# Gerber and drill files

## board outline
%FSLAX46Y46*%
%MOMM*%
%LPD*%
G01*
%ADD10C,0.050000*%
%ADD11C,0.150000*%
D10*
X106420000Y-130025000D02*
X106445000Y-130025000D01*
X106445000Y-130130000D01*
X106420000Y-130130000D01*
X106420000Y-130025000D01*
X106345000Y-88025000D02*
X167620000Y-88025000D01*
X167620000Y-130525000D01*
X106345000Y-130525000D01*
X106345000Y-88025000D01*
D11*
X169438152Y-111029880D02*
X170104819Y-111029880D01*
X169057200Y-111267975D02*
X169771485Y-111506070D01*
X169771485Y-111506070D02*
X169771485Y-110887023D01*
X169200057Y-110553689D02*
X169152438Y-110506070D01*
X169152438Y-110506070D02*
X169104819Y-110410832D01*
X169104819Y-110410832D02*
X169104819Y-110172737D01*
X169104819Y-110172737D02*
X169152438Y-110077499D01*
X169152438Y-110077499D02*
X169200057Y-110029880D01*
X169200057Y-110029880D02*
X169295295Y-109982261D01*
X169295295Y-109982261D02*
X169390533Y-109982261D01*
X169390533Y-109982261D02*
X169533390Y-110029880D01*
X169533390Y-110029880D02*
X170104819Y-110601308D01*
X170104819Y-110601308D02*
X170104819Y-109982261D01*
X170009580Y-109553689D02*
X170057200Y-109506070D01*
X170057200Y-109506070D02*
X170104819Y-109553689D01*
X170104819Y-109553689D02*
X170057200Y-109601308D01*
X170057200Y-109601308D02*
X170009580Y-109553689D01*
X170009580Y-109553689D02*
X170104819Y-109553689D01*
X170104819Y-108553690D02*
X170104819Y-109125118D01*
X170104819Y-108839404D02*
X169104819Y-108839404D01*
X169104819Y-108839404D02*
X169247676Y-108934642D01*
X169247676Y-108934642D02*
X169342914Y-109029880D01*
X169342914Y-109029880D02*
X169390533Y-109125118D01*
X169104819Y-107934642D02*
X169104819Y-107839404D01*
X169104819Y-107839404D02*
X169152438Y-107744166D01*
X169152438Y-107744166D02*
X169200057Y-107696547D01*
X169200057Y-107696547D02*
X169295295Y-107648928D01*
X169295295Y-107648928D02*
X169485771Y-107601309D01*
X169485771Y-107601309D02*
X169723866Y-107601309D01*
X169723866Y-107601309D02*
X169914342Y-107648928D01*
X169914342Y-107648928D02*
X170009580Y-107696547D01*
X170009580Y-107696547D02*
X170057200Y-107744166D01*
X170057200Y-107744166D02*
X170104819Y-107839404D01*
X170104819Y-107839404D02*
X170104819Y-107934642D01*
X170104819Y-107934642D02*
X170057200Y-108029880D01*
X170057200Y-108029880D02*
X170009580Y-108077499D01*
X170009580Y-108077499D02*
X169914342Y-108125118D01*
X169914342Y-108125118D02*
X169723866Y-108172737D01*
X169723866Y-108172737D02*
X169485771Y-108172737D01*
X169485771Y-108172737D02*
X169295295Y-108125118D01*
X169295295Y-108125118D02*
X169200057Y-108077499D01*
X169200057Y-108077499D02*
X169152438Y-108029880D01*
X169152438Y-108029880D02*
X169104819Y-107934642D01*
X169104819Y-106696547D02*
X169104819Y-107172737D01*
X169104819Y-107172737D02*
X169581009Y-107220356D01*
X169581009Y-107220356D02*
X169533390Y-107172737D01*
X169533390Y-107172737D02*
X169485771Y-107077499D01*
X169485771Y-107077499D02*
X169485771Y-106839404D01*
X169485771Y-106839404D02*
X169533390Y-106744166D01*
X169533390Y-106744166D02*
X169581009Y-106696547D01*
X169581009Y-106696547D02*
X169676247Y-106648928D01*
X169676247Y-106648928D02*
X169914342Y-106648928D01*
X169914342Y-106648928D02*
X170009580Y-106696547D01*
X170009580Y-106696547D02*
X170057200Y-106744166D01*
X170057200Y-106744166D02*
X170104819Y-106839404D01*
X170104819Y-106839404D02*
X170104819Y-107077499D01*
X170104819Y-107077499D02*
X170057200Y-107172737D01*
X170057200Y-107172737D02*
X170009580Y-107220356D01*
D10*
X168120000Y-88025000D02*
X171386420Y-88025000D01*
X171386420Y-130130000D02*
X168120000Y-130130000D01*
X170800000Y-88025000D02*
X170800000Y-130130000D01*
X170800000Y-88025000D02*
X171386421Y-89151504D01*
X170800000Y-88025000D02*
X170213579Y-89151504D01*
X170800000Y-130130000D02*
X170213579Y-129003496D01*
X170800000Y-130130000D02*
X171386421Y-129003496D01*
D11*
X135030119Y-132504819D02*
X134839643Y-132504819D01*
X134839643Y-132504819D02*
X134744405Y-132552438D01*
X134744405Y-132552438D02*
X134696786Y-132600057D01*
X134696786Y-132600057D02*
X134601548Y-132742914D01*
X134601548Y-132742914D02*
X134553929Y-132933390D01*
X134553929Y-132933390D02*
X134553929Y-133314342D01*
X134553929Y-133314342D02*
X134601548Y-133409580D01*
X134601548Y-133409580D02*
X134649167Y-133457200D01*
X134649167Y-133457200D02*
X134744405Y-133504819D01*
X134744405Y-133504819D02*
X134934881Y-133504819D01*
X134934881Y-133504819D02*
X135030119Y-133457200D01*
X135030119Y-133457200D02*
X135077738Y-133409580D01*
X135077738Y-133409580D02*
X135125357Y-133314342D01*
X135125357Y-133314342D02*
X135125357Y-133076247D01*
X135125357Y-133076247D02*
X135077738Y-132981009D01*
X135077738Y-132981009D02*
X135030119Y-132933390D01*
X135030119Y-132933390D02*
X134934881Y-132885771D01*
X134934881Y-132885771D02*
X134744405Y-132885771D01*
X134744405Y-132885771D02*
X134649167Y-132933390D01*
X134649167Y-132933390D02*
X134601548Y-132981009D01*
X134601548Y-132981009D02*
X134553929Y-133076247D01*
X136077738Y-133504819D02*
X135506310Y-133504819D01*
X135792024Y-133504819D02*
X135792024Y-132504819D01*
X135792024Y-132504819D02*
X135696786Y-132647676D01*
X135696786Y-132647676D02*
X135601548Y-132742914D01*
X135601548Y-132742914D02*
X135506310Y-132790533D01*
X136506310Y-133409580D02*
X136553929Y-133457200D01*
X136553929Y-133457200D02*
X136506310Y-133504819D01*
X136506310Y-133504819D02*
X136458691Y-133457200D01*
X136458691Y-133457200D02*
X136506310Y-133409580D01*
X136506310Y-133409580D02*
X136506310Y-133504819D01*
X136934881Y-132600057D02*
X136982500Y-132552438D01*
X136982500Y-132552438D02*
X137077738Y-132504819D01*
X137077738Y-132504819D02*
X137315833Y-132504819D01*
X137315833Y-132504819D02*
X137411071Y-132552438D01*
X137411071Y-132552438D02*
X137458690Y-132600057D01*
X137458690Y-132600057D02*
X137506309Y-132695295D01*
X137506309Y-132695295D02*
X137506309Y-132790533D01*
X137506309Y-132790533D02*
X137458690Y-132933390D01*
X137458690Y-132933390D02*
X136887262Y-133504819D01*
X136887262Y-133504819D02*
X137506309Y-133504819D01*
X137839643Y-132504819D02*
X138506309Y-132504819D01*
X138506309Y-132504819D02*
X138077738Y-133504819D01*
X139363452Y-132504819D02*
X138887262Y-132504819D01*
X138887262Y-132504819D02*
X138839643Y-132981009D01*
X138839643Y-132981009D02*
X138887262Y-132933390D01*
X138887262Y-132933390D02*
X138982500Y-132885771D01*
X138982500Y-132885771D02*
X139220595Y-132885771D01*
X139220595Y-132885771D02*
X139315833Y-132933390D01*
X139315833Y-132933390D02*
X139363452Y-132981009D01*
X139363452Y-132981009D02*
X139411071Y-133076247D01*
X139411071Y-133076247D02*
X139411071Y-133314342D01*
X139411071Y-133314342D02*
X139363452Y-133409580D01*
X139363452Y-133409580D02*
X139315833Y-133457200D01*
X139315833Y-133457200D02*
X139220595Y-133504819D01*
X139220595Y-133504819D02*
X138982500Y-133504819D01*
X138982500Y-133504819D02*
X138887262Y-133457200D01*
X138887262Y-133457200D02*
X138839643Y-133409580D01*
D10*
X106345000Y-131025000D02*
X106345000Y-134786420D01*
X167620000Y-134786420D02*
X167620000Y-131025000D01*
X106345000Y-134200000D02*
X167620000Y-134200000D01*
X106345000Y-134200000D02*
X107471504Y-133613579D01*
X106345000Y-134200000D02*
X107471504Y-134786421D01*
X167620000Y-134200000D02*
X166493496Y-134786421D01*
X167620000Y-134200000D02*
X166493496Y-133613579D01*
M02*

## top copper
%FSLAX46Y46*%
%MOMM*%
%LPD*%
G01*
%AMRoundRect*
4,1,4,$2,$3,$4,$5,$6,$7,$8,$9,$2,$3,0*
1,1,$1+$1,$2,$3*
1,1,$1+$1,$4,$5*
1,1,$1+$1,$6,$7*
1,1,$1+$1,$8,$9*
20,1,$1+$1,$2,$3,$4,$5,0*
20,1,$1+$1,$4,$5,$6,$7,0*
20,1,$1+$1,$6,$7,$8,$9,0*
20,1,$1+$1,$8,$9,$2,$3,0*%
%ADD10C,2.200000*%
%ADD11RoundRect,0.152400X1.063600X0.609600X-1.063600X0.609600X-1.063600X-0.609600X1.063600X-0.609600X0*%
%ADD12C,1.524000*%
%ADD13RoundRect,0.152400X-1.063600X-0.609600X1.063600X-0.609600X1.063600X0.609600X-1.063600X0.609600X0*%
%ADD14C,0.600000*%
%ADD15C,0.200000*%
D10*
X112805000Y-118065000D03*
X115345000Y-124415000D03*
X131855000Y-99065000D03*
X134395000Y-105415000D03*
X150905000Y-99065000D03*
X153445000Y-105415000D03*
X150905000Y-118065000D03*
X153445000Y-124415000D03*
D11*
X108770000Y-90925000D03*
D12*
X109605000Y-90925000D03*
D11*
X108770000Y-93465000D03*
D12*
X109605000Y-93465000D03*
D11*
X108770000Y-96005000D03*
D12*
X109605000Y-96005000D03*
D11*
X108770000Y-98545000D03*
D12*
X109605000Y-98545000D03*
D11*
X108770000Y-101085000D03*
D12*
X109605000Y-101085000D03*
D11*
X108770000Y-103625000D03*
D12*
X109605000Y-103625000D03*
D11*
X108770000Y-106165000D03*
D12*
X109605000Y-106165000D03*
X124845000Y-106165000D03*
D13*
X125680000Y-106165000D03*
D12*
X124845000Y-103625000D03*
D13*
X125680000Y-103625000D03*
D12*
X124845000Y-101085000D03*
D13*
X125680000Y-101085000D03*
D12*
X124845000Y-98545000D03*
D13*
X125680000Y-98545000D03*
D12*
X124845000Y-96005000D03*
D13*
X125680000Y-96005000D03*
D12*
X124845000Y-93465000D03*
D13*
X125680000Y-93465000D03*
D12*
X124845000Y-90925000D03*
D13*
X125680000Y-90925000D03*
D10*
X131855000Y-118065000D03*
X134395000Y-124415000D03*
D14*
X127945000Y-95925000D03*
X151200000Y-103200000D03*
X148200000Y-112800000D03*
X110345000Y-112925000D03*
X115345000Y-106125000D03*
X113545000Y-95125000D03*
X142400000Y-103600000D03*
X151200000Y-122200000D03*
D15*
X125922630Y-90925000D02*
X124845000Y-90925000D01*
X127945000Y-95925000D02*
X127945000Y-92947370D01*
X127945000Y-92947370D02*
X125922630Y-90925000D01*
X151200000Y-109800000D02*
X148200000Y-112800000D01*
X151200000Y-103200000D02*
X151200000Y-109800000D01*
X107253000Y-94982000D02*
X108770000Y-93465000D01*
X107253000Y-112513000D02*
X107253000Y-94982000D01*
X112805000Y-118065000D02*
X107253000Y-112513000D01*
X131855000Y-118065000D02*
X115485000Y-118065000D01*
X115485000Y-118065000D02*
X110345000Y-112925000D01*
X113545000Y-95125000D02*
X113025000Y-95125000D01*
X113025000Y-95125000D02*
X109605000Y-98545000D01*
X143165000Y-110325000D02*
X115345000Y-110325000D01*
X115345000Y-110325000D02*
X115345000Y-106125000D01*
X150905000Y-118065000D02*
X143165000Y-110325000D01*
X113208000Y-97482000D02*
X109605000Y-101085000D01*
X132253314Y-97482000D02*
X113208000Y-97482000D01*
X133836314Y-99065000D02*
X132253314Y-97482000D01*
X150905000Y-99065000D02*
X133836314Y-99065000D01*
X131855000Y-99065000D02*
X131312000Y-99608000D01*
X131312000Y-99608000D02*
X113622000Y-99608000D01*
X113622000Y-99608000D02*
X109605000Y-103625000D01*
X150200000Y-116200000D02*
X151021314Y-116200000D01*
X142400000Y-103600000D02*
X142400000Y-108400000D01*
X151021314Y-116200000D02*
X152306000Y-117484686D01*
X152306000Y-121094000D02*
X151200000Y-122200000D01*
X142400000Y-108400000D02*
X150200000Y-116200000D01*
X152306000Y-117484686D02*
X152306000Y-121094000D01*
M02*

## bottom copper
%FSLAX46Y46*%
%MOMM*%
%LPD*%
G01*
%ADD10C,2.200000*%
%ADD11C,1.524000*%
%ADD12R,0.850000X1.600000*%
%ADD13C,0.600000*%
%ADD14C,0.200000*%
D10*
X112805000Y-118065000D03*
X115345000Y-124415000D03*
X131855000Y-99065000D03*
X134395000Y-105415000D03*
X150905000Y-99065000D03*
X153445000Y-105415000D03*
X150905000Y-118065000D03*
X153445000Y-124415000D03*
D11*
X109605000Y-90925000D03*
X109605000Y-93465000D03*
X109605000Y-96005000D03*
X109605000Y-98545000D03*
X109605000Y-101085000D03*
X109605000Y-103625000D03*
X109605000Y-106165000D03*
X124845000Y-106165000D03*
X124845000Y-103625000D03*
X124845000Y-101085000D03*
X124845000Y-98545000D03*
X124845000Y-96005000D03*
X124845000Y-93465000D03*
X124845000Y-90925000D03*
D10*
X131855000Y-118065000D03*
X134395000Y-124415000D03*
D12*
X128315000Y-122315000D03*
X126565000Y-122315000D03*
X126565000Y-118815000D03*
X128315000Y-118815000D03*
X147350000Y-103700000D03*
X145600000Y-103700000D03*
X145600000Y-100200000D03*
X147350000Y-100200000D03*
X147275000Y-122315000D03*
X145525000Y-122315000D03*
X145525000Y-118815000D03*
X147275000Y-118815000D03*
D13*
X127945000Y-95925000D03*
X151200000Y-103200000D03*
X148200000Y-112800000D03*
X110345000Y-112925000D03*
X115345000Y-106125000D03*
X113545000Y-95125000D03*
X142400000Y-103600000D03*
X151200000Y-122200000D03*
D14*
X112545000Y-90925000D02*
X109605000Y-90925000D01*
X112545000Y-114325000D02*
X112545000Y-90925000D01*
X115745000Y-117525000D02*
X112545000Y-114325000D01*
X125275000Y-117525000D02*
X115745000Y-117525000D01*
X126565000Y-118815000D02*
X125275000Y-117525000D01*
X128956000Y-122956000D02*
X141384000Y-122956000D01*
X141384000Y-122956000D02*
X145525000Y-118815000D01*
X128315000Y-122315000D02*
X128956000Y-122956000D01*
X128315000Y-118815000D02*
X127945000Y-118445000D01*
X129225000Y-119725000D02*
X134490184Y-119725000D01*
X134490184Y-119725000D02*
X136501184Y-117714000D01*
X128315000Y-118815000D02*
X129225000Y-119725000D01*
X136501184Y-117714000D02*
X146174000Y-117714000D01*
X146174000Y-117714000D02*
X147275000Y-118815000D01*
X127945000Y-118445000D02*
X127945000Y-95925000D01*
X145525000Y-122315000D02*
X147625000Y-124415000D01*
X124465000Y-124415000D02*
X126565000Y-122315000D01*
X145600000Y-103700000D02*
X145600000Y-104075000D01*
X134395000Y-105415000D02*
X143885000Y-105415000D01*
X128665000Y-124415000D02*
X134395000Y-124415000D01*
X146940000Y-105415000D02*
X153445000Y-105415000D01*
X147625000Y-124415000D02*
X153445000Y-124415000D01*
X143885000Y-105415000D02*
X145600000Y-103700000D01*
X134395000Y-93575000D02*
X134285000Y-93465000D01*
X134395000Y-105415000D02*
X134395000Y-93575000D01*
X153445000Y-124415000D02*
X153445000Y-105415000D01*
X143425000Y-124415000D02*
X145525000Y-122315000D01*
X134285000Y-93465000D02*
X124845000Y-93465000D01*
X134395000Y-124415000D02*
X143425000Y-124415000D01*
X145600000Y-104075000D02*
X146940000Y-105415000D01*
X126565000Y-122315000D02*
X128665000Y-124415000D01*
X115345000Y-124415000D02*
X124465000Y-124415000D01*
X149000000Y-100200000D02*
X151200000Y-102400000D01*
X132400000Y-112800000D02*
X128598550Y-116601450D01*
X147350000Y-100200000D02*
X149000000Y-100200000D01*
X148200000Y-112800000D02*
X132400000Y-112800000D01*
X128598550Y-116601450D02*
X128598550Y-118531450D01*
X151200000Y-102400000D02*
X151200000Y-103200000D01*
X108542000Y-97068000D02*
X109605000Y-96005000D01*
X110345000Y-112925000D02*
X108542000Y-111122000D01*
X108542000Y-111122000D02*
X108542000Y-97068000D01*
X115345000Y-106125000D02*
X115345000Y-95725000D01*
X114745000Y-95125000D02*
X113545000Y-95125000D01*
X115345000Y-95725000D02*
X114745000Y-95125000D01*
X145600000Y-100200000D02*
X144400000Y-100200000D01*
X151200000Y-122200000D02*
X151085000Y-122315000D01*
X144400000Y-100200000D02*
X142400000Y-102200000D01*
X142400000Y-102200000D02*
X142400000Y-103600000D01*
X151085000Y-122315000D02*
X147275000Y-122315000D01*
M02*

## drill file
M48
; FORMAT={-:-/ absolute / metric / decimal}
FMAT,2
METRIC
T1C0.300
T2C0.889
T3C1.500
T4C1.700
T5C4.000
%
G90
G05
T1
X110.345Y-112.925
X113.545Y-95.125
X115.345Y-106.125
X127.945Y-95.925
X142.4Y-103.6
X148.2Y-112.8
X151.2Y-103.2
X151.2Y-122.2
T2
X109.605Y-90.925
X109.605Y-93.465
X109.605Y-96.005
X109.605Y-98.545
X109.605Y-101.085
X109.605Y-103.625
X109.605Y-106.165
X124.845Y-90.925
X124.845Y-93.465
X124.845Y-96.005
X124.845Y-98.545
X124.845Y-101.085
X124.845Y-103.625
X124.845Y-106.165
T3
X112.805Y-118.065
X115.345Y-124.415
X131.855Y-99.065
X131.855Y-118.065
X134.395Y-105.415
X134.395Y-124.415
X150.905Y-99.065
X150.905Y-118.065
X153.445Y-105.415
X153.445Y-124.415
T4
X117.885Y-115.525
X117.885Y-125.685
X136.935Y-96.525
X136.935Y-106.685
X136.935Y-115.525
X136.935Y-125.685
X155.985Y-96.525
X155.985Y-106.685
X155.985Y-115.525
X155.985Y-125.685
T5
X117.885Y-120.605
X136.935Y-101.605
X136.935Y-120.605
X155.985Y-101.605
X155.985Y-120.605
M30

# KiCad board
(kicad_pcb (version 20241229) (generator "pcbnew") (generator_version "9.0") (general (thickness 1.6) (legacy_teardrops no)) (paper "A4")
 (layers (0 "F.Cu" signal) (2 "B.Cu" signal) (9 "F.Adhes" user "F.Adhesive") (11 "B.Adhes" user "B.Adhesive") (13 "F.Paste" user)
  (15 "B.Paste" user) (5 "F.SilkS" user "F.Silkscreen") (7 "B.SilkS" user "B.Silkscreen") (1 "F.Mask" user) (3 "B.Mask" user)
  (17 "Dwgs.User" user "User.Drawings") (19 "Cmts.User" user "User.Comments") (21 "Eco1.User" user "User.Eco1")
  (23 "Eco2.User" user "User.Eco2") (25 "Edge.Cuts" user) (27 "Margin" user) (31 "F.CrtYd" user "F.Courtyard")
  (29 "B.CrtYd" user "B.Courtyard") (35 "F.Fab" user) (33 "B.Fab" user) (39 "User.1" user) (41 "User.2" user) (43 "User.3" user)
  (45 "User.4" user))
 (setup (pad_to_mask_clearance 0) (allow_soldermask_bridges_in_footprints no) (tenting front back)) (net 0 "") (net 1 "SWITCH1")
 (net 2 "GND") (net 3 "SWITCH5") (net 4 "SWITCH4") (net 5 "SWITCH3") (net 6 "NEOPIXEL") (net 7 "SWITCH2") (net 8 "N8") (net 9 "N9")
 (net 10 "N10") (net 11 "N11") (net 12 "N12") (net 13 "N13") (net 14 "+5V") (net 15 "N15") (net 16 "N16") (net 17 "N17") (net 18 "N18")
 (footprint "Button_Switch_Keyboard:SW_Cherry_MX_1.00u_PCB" (layer "F.Cu") (at 112.805 118.065 90)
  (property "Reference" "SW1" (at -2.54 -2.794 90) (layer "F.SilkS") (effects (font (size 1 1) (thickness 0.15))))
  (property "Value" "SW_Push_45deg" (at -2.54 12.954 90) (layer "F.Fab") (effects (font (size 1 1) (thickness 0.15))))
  (pad "" np_thru_hole circle (at -7.62 5.08 90) (size 1.7 1.7) (drill 1.7) (layers "*.Cu" "*.Mask"))
  (pad "" np_thru_hole circle (at -2.54 5.08 90) (size 4 4) (drill 4) (layers "*.Cu" "*.Mask"))
  (pad "" np_thru_hole circle (at 2.54 5.08 90) (size 1.7 1.7) (drill 1.7) (layers "*.Cu" "*.Mask"))
  (pad "1" thru_hole circle (at 0 0 90) (size 2.2 2.2) (drill 1.5) (layers "*.Cu" "*.Mask") (remove_unused_layers no) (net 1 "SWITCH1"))
  (pad "2" thru_hole circle (at -6.35 2.54 90) (size 2.2 2.2) (drill 1.5) (layers "*.Cu" "*.Mask") (remove_unused_layers no) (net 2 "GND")))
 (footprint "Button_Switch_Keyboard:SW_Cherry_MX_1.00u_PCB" (layer "F.Cu") (at 131.855 99.065 90)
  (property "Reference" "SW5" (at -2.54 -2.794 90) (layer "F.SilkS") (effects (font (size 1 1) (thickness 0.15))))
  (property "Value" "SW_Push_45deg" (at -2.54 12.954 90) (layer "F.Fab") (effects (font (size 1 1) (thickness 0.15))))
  (pad "" np_thru_hole circle (at -7.62 5.08 90) (size 1.7 1.7) (drill 1.7) (layers "*.Cu" "*.Mask"))
  (pad "" np_thru_hole circle (at -2.54 5.08 90) (size 4 4) (drill 4) (layers "*.Cu" "*.Mask"))
  (pad "" np_thru_hole circle (at 2.54 5.08 90) (size 1.7 1.7) (drill 1.7) (layers "*.Cu" "*.Mask"))
  (pad "1" thru_hole circle (at 0 0 90) (size 2.2 2.2) (drill 1.5) (layers "*.Cu" "*.Mask") (remove_unused_layers no) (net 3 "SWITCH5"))
  (pad "2" thru_hole circle (at -6.35 2.54 90) (size 2.2 2.2) (drill 1.5) (layers "*.Cu" "*.Mask") (remove_unused_layers no) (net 2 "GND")))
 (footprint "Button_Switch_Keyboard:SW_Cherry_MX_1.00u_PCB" (layer "F.Cu") (at 150.905 99.065 90)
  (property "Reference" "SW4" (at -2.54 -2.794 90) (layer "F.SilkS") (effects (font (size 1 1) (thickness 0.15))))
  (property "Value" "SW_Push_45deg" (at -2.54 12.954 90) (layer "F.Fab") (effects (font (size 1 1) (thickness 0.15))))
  (pad "" np_thru_hole circle (at -7.62 5.08 90) (size 1.7 1.7) (drill 1.7) (layers "*.Cu" "*.Mask"))
  (pad "" np_thru_hole circle (at -2.54 5.08 90) (size 4 4) (drill 4) (layers "*.Cu" "*.Mask"))
  (pad "" np_thru_hole circle (at 2.54 5.08 90) (size 1.7 1.7) (drill 1.7) (layers "*.Cu" "*.Mask"))
  (pad "1" thru_hole circle (at 0 0 90) (size 2.2 2.2) (drill 1.5) (layers "*.Cu" "*.Mask") (remove_unused_layers no) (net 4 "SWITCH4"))
  (pad "2" thru_hole circle (at -6.35 2.54 90) (size 2.2 2.2) (drill 1.5) (layers "*.Cu" "*.Mask") (remove_unused_layers no) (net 2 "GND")))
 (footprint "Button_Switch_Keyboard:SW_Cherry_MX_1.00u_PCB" (layer "F.Cu") (at 150.905 118.065 90)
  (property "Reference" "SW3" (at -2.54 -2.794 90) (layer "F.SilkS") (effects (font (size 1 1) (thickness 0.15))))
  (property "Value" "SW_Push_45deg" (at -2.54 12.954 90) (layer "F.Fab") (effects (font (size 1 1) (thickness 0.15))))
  (pad "" np_thru_hole circle (at -7.62 5.08 90) (size 1.7 1.7) (drill 1.7) (layers "*.Cu" "*.Mask"))
  (pad "" np_thru_hole circle (at -2.54 5.08 90) (size 4 4) (drill 4) (layers "*.Cu" "*.Mask"))
  (pad "" np_thru_hole circle (at 2.54 5.08 90) (size 1.7 1.7) (drill 1.7) (layers "*.Cu" "*.Mask"))
  (pad "1" thru_hole circle (at 0 0 90) (size 2.2 2.2) (drill 1.5) (layers "*.Cu" "*.Mask") (remove_unused_layers no) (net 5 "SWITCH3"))
  (pad "2" thru_hole circle (at -6.35 2.54 90) (size 2.2 2.2) (drill 1.5) (layers "*.Cu" "*.Mask") (remove_unused_layers no) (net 2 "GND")))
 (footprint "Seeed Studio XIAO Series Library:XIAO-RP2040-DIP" (layer "F.Cu") (at 117.225 98.545)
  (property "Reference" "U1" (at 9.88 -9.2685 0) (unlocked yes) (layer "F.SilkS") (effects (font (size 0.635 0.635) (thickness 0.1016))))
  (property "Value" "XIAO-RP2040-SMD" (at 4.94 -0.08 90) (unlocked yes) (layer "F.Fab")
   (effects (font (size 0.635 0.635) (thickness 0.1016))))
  (pad "1" smd roundrect (at -8.455 -7.62 180) (size 2.432 1.524) (layers "F.Cu" "F.Mask") (roundrect_rratio 0.1) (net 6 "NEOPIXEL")
   (thermal_bridge_angle 45))
  (pad "1" thru_hole circle (at -7.62 -7.62 180) (size 1.524 1.524) (drill 0.889) (layers "*.Cu" "*.Mask") (remove_unused_layers no)
   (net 6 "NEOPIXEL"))
  (pad "2" smd roundrect (at -8.455 -5.08 180) (size 2.432 1.524) (layers "F.Cu" "F.Mask") (roundrect_rratio 0.1) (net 1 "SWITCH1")
   (thermal_bridge_angle 45))
  (pad "2" thru_hole circle (at -7.62 -5.08 180) (size 1.524 1.524) (drill 0.889) (layers "*.Cu" "*.Mask") (remove_unused_layers no)
   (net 1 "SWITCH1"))
  (pad "3" smd roundrect (at -8.455 -2.54 180) (size 2.432 1.524) (layers "F.Cu" "F.Mask") (roundrect_rratio 0.1) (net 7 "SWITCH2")
   (thermal_bridge_angle 45))
  (pad "3" thru_hole circle (at -7.62 -2.54 180) (size 1.524 1.524) (drill 0.889) (layers "*.Cu" "*.Mask") (remove_unused_layers no)
   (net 7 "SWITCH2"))
  (pad "4" smd roundrect (at -8.455 0 180) (size 2.432 1.524) (layers "F.Cu" "F.Mask") (roundrect_rratio 0.1) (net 5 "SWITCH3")
   (thermal_bridge_angle 45))
  (pad "4" thru_hole circle (at -7.62 0 180) (size 1.524 1.524) (drill 0.889) (layers "*.Cu" "*.Mask") (remove_unused_layers no)
   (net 5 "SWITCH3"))
  (pad "5" smd roundrect (at -8.455 2.54 180) (size 2.432 1.524) (layers "F.Cu" "F.Mask") (roundrect_rratio 0.1) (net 4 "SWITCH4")
   (thermal_bridge_angle 45))
  (pad "5" thru_hole circle (at -7.62 2.54 180) (size 1.524 1.524) (drill 0.889) (layers "*.Cu" "*.Mask") (remove_unused_layers no)
   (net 4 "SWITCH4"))
  (pad "6" smd roundrect (at -8.455 5.08 180) (size 2.432 1.524) (layers "F.Cu" "F.Mask") (roundrect_rratio 0.1) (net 3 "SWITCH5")
   (thermal_bridge_angle 45))
  (pad "6" thru_hole circle (at -7.62 5.08 180) (size 1.524 1.524) (drill 0.889) (layers "*.Cu" "*.Mask") (remove_unused_layers no)
   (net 3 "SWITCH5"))
  (pad "7" smd roundrect (at -8.455 7.62 180) (size 2.432 1.524) (layers "F.Cu" "F.Mask") (roundrect_rratio 0.1) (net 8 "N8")
   (thermal_bridge_angle 45))
  (pad "7" thru_hole circle (at -7.62 7.62 180) (size 1.524 1.524) (drill 0.889) (layers "*.Cu" "*.Mask") (remove_unused_layers no)
   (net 8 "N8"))
  (pad "8" thru_hole circle (at 7.62 7.62) (size 1.524 1.524) (drill 0.889) (layers "*.Cu" "*.Mask") (remove_unused_layers no) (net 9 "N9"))
  (pad "8" smd roundrect (at 8.455 7.62) (size 2.432 1.524) (layers "F.Cu" "F.Mask") (roundrect_rratio 0.1) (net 9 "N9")
   (thermal_bridge_angle 45))
  (pad "9" thru_hole circle (at 7.62 5.08) (size 1.524 1.524) (drill 0.889) (layers "*.Cu" "*.Mask") (remove_unused_layers no)
   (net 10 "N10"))
  (pad "9" smd roundrect (at 8.455 5.08) (size 2.432 1.524) (layers "F.Cu" "F.Mask") (roundrect_rratio 0.1) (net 10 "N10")
   (thermal_bridge_angle 45))
  (pad "10" thru_hole circle (at 7.62 2.54) (size 1.524 1.524) (drill 0.889) (layers "*.Cu" "*.Mask") (remove_unused_layers no)
   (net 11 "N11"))
  (pad "10" smd roundrect (at 8.455 2.54) (size 2.432 1.524) (layers "F.Cu" "F.Mask") (roundrect_rratio 0.1) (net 11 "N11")
   (thermal_bridge_angle 45))
  (pad "11" thru_hole circle (at 7.62 0) (size 1.524 1.524) (drill 0.889) (layers "*.Cu" "*.Mask") (remove_unused_layers no) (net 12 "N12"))
  (pad "11" smd roundrect (at 8.455 0) (size 2.432 1.524) (layers "F.Cu" "F.Mask") (roundrect_rratio 0.1) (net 12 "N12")
   (thermal_bridge_angle 45))
  (pad "12" thru_hole circle (at 7.62 -2.54) (size 1.524 1.524) (drill 0.889) (layers "*.Cu" "*.Mask") (remove_unused_layers no)
   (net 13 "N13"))
  (pad "12" smd roundrect (at 8.455 -2.54) (size 2.432 1.524) (layers "F.Cu" "F.Mask") (roundrect_rratio 0.1) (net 13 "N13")
   (thermal_bridge_angle 45))
  (pad "13" thru_hole circle (at 7.62 -5.08) (size 1.524 1.524) (drill 0.889) (layers "*.Cu" "*.Mask") (remove_unused_layers no)
   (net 2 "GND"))
  (pad "13" smd roundrect (at 8.455 -5.08) (size 2.432 1.524) (layers "F.Cu" "F.Mask") (roundrect_rratio 0.1) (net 2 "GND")
   (thermal_bridge_angle 45))
  (pad "14" thru_hole circle (at 7.62 -7.62) (size 1.524 1.524) (drill 0.889) (layers "*.Cu" "*.Mask") (remove_unused_layers no)
   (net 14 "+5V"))
  (pad "14" smd roundrect (at 8.455 -7.62) (size 2.432 1.524) (layers "F.Cu" "F.Mask") (roundrect_rratio 0.1) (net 14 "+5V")
   (thermal_bridge_angle 45)))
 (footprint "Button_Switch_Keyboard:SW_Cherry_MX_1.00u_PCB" (layer "F.Cu") (at 131.855 118.065 90)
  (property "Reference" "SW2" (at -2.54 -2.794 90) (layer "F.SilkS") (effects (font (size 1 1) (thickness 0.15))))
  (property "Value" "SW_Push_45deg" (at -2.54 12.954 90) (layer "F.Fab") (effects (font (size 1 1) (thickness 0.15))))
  (pad "" np_thru_hole circle (at -7.62 5.08 90) (size 1.7 1.7) (drill 1.7) (layers "*.Cu" "*.Mask"))
  (pad "" np_thru_hole circle (at -2.54 5.08 90) (size 4 4) (drill 4) (layers "*.Cu" "*.Mask"))
  (pad "" np_thru_hole circle (at 2.54 5.08 90) (size 1.7 1.7) (drill 1.7) (layers "*.Cu" "*.Mask"))
  (pad "1" thru_hole circle (at 0 0 90) (size 2.2 2.2) (drill 1.5) (layers "*.Cu" "*.Mask") (remove_unused_layers no) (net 7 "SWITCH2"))
  (pad "2" thru_hole circle (at -6.35 2.54 90) (size 2.2 2.2) (drill 1.5) (layers "*.Cu" "*.Mask") (remove_unused_layers no) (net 2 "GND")))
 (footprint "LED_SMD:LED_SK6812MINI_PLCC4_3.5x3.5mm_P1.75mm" (layer "B.Cu") (at 127.44 120.565 90)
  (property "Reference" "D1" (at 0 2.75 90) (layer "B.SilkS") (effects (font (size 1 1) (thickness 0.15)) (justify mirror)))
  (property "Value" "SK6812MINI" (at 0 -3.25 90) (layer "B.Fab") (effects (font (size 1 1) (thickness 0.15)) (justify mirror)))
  (pad "1" smd rect (at -1.75 0.875 90) (size 1.6 0.85) (layers "B.Cu" "B.Mask" "B.Paste") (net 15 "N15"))
  (pad "2" smd rect (at -1.75 -0.875 90) (size 1.6 0.85) (layers "B.Cu" "B.Mask" "B.Paste") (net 2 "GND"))
  (pad "3" smd rect (at 1.75 -0.875 90) (size 1.6 0.85) (layers "B.Cu" "B.Mask" "B.Paste") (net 6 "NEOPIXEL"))
  (pad "4" smd rect (at 1.75 0.875 90) (size 1.6 0.85) (layers "B.Cu" "B.Mask" "B.Paste") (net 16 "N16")))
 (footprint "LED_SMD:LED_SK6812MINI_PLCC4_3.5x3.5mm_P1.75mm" (layer "B.Cu") (at 146.475 101.95 90)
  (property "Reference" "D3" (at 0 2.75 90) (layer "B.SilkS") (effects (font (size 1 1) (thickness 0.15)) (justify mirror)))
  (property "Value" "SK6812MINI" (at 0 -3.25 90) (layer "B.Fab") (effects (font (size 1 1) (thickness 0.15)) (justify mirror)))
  (pad "1" smd rect (at -1.75 0.875 90) (size 1.6 0.85) (layers "B.Cu" "B.Mask" "B.Paste") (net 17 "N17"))
  (pad "2" smd rect (at -1.75 -0.875 90) (size 1.6 0.85) (layers "B.Cu" "B.Mask" "B.Paste") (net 2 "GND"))
  (pad "3" smd rect (at 1.75 -0.875 90) (size 1.6 0.85) (layers "B.Cu" "B.Mask" "B.Paste") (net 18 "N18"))
  (pad "4" smd rect (at 1.75 0.875 90) (size 1.6 0.85) (layers "B.Cu" "B.Mask" "B.Paste") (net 16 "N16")))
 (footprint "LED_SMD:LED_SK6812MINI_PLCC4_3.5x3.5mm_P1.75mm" (layer "B.Cu") (at 146.4 120.565 90)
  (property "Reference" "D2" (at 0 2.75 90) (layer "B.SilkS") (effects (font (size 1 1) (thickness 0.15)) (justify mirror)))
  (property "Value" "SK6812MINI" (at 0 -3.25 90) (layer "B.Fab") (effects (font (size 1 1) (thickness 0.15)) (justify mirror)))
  (pad "1" smd rect (at -1.75 0.875 90) (size 1.6 0.85) (layers "B.Cu" "B.Mask" "B.Paste") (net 18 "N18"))
  (pad "2" smd rect (at -1.75 -0.875 90) (size 1.6 0.85) (layers "B.Cu" "B.Mask" "B.Paste") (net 2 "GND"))
  (pad "3" smd rect (at 1.75 -0.875 90) (size 1.6 0.85) (layers "B.Cu" "B.Mask" "B.Paste") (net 15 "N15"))
  (pad "4" smd rect (at 1.75 0.875 90) (size 1.6 0.85) (layers "B.Cu" "B.Mask" "B.Paste") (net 14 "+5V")))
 (gr_rect (start 106.42 130.025) (end 106.445 130.13) (stroke (width 0.05) (type default)) (fill no) (layer "Edge.Cuts"))
 (gr_rect (start 106.345 88.025) (end 167.62 130.525) (stroke (width 0.05) (type default)) (fill no) (layer "Edge.Cuts"))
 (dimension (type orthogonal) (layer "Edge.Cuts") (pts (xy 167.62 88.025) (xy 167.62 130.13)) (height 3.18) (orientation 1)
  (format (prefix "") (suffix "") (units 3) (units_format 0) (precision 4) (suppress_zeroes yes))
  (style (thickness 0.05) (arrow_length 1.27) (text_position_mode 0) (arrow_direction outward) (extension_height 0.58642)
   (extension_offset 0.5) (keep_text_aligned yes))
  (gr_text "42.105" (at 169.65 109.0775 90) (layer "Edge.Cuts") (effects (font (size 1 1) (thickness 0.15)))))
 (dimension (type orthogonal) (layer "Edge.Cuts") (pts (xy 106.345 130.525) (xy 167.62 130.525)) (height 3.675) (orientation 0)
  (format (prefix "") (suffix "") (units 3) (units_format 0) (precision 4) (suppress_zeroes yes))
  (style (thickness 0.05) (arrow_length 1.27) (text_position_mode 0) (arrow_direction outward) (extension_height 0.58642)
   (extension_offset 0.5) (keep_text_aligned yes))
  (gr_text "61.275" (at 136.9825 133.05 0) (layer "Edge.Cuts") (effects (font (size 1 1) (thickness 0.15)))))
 (segment (start 112.545 90.925) (end 109.605 90.925) (width 0.2) (layer "B.Cu") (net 6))
 (segment (start 112.545 114.325) (end 112.545 90.925) (width 0.2) (layer "B.Cu") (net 6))
 (segment (start 115.745 117.525) (end 112.545 114.325) (width 0.2) (layer "B.Cu") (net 6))
 (segment (start 125.275 117.525) (end 115.745 117.525) (width 0.2) (layer "B.Cu") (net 6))
 (segment (start 126.565 118.815) (end 125.275 117.525) (width 0.2) (layer "B.Cu") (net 6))
 (segment (start 128.956 122.956) (end 141.384 122.956) (width 0.2) (layer "B.Cu") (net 15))
 (segment (start 141.384 122.956) (end 145.525 118.815) (width 0.2) (layer "B.Cu") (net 15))
 (segment (start 128.315 122.315) (end 128.956 122.956) (width 0.2) (layer "B.Cu") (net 15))
 (segment (start 125.92263 90.925) (end 124.845 90.925) (width 0.2) (layer "F.Cu") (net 14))
 (segment (start 127.945 95.925) (end 127.945 92.94737) (width 0.2) (layer "F.Cu") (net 14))
 (segment (start 127.945 92.94737) (end 125.92263 90.925) (width 0.2) (layer "F.Cu") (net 14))
 (via (at 127.945 95.925) (size 0.6) (drill 0.3) (layers "F.Cu" "B.Cu") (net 14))
 (segment (start 128.315 118.815) (end 127.945 118.445) (width 0.2) (layer "B.Cu") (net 14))
 (segment (start 129.225 119.725) (end 134.490184 119.725) (width 0.2) (layer "B.Cu") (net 14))
 (segment (start 134.490184 119.725) (end 136.501184 117.714) (width 0.2) (layer "B.Cu") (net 14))
 (segment (start 128.315 118.815) (end 129.225 119.725) (width 0.2) (layer "B.Cu") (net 14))
 (segment (start 136.501184 117.714) (end 146.174 117.714) (width 0.2) (layer "B.Cu") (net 14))
 (segment (start 146.174 117.714) (end 147.275 118.815) (width 0.2) (layer "B.Cu") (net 14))
 (segment (start 127.945 118.445) (end 127.945 95.925) (width 0.2) (layer "B.Cu") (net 14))
 (segment (start 145.525 122.315) (end 147.625 124.415) (width 0.2) (layer "B.Cu") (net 2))
 (segment (start 124.465 124.415) (end 126.565 122.315) (width 0.2) (layer "B.Cu") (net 2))
 (segment (start 145.6 103.7) (end 145.6 104.075) (width 0.2) (layer "B.Cu") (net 2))
 (segment (start 134.395 105.415) (end 143.885 105.415) (width 0.2) (layer "B.Cu") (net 2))
 (segment (start 128.665 124.415) (end 134.395 124.415) (width 0.2) (layer "B.Cu") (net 2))
 (segment (start 146.94 105.415) (end 153.445 105.415) (width 0.2) (layer "B.Cu") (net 2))
 (segment (start 147.625 124.415) (end 153.445 124.415) (width 0.2) (layer "B.Cu") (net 2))
 (segment (start 143.885 105.415) (end 145.6 103.7) (width 0.2) (layer "B.Cu") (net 2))
 (segment (start 134.395 93.575) (end 134.285 93.465) (width 0.2) (layer "B.Cu") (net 2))
 (segment (start 134.395 105.415) (end 134.395 93.575) (width 0.2) (layer "B.Cu") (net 2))
 (segment (start 153.445 124.415) (end 153.445 105.415) (width 0.2) (layer "B.Cu") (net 2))
 (segment (start 143.425 124.415) (end 145.525 122.315) (width 0.2) (layer "B.Cu") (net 2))
 (segment (start 134.285 93.465) (end 124.845 93.465) (width 0.2) (layer "B.Cu") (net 2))
 (segment (start 134.395 124.415) (end 143.425 124.415) (width 0.2) (layer "B.Cu") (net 2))
 (segment (start 145.6 104.075) (end 146.94 105.415) (width 0.2) (layer "B.Cu") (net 2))
 (segment (start 126.565 122.315) (end 128.665 124.415) (width 0.2) (layer "B.Cu") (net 2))
 (segment (start 115.345 124.415) (end 124.465 124.415) (width 0.2) (layer "B.Cu") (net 2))
 (segment (start 151.2 109.8) (end 148.2 112.8) (width 0.2) (layer "F.Cu") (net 16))
 (segment (start 151.2 103.2) (end 151.2 109.8) (width 0.2) (layer "F.Cu") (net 16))
 (via (at 151.2 103.2) (size 0.6) (drill 0.3) (layers "F.Cu" "B.Cu") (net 16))
 (via (at 148.2 112.8) (size 0.6) (drill 0.3) (layers "F.Cu" "B.Cu") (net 16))
 (segment (start 149 100.2) (end 151.2 102.4) (width 0.2) (layer "B.Cu") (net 16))
 (segment (start 132.4 112.8) (end 128.59855 116.60145) (width 0.2) (layer "B.Cu") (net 16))
 (segment (start 147.35 100.2) (end 149 100.2) (width 0.2) (layer "B.Cu") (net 16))
 (segment (start 148.2 112.8) (end 132.4 112.8) (width 0.2) (layer "B.Cu") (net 16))
 (segment (start 128.59855 116.60145) (end 128.59855 118.53145) (width 0.2) (layer "B.Cu") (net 16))
 (segment (start 151.2 102.4) (end 151.2 103.2) (width 0.2) (layer "B.Cu") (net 16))
 (segment (start 107.253 94.982) (end 108.77 93.465) (width 0.2) (layer "F.Cu") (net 1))
 (segment (start 107.253 112.513) (end 107.253 94.982) (width 0.2) (layer "F.Cu") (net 1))
 (segment (start 112.805 118.065) (end 107.253 112.513) (width 0.2) (layer "F.Cu") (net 1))
 (segment (start 131.855 118.065) (end 115.485 118.065) (width 0.2) (layer "F.Cu") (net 7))
 (segment (start 115.485 118.065) (end 110.345 112.925) (width 0.2) (layer "F.Cu") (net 7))
 (via (at 110.345 112.925) (size 0.6) (drill 0.3) (layers "F.Cu" "B.Cu") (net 7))
 (segment (start 108.542 97.068) (end 109.605 96.005) (width 0.2) (layer "B.Cu") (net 7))
 (segment (start 110.345 112.925) (end 108.542 111.122) (width 0.2) (layer "B.Cu") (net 7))
 (segment (start 108.542 111.122) (end 108.542 97.068) (width 0.2) (layer "B.Cu") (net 7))
 (segment (start 113.545 95.125) (end 113.025 95.125) (width 0.2) (layer "F.Cu") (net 5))
 (segment (start 113.025 95.125) (end 109.605 98.545) (width 0.2) (layer "F.Cu") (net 5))
 (segment (start 143.165 110.325) (end 115.345 110.325) (width 0.2) (layer "F.Cu") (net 5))
 (segment (start 115.345 110.325) (end 115.345 106.125) (width 0.2) (layer "F.Cu") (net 5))
 (segment (start 150.905 118.065) (end 143.165 110.325) (width 0.2) (layer "F.Cu") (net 5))
 (via (at 115.345 106.125) (size 0.6) (drill 0.3) (layers "F.Cu" "B.Cu") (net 5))
 (via (at 113.545 95.125) (size 0.6) (drill 0.3) (layers "F.Cu" "B.Cu") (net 5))
 (segment (start 115.345 106.125) (end 115.345 95.725) (width 0.2) (layer "B.Cu") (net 5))
 (segment (start 114.745 95.125) (end 113.545 95.125) (width 0.2) (layer "B.Cu") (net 5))
 (segment (start 115.345 95.725) (end 114.745 95.125) (width 0.2) (layer "B.Cu") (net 5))
 (segment (start 113.208 97.482) (end 109.605 101.085) (width 0.2) (layer "F.Cu") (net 4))
 (segment (start 132.253314 97.482) (end 113.208 97.482) (width 0.2) (layer "F.Cu") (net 4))
 (segment (start 133.836314 99.065) (end 132.253314 97.482) (width 0.2) (layer "F.Cu") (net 4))
 (segment (start 150.905 99.065) (end 133.836314 99.065) (width 0.2) (layer "F.Cu") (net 4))
 (segment (start 131.855 99.065) (end 131.312 99.608) (width 0.2) (layer "F.Cu") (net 3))
 (segment (start 131.312 99.608) (end 113.622 99.608) (width 0.2) (layer "F.Cu") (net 3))
 (segment (start 113.622 99.608) (end 109.605 103.625) (width 0.2) (layer "F.Cu") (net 3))
 (segment (start 150.2 116.2) (end 151.021314 116.2) (width 0.2) (layer "F.Cu") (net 18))
 (segment (start 142.4 103.6) (end 142.4 108.4) (width 0.2) (layer "F.Cu") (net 18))
 (segment (start 151.021314 116.2) (end 152.306 117.484686) (width 0.2) (layer "F.Cu") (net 18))
 (segment (start 152.306 121.094) (end 151.2 122.2) (width 0.2) (layer "F.Cu") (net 18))
 (segment (start 142.4 108.4) (end 150.2 116.2) (width 0.2) (layer "F.Cu") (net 18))
 (segment (start 152.306 117.484686) (end 152.306 121.094) (width 0.2) (layer "F.Cu") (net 18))
 (via (at 142.4 103.6) (size 0.6) (drill 0.3) (layers "F.Cu" "B.Cu") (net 18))
 (via (at 151.2 122.2) (size 0.6) (drill 0.3) (layers "F.Cu" "B.Cu") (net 18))
 (segment (start 145.6 100.2) (end 144.4 100.2) (width 0.2) (layer "B.Cu") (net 18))
 (segment (start 151.2 122.2) (end 151.085 122.315) (width 0.2) (layer "B.Cu") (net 18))
 (segment (start 144.4 100.2) (end 142.4 102.2) (width 0.2) (layer "B.Cu") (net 18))
 (segment (start 142.4 102.2) (end 142.4 103.6) (width 0.2) (layer "B.Cu") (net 18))
 (segment (start 151.085 122.315) (end 147.275 122.315) (width 0.2) (layer "B.Cu") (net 18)))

